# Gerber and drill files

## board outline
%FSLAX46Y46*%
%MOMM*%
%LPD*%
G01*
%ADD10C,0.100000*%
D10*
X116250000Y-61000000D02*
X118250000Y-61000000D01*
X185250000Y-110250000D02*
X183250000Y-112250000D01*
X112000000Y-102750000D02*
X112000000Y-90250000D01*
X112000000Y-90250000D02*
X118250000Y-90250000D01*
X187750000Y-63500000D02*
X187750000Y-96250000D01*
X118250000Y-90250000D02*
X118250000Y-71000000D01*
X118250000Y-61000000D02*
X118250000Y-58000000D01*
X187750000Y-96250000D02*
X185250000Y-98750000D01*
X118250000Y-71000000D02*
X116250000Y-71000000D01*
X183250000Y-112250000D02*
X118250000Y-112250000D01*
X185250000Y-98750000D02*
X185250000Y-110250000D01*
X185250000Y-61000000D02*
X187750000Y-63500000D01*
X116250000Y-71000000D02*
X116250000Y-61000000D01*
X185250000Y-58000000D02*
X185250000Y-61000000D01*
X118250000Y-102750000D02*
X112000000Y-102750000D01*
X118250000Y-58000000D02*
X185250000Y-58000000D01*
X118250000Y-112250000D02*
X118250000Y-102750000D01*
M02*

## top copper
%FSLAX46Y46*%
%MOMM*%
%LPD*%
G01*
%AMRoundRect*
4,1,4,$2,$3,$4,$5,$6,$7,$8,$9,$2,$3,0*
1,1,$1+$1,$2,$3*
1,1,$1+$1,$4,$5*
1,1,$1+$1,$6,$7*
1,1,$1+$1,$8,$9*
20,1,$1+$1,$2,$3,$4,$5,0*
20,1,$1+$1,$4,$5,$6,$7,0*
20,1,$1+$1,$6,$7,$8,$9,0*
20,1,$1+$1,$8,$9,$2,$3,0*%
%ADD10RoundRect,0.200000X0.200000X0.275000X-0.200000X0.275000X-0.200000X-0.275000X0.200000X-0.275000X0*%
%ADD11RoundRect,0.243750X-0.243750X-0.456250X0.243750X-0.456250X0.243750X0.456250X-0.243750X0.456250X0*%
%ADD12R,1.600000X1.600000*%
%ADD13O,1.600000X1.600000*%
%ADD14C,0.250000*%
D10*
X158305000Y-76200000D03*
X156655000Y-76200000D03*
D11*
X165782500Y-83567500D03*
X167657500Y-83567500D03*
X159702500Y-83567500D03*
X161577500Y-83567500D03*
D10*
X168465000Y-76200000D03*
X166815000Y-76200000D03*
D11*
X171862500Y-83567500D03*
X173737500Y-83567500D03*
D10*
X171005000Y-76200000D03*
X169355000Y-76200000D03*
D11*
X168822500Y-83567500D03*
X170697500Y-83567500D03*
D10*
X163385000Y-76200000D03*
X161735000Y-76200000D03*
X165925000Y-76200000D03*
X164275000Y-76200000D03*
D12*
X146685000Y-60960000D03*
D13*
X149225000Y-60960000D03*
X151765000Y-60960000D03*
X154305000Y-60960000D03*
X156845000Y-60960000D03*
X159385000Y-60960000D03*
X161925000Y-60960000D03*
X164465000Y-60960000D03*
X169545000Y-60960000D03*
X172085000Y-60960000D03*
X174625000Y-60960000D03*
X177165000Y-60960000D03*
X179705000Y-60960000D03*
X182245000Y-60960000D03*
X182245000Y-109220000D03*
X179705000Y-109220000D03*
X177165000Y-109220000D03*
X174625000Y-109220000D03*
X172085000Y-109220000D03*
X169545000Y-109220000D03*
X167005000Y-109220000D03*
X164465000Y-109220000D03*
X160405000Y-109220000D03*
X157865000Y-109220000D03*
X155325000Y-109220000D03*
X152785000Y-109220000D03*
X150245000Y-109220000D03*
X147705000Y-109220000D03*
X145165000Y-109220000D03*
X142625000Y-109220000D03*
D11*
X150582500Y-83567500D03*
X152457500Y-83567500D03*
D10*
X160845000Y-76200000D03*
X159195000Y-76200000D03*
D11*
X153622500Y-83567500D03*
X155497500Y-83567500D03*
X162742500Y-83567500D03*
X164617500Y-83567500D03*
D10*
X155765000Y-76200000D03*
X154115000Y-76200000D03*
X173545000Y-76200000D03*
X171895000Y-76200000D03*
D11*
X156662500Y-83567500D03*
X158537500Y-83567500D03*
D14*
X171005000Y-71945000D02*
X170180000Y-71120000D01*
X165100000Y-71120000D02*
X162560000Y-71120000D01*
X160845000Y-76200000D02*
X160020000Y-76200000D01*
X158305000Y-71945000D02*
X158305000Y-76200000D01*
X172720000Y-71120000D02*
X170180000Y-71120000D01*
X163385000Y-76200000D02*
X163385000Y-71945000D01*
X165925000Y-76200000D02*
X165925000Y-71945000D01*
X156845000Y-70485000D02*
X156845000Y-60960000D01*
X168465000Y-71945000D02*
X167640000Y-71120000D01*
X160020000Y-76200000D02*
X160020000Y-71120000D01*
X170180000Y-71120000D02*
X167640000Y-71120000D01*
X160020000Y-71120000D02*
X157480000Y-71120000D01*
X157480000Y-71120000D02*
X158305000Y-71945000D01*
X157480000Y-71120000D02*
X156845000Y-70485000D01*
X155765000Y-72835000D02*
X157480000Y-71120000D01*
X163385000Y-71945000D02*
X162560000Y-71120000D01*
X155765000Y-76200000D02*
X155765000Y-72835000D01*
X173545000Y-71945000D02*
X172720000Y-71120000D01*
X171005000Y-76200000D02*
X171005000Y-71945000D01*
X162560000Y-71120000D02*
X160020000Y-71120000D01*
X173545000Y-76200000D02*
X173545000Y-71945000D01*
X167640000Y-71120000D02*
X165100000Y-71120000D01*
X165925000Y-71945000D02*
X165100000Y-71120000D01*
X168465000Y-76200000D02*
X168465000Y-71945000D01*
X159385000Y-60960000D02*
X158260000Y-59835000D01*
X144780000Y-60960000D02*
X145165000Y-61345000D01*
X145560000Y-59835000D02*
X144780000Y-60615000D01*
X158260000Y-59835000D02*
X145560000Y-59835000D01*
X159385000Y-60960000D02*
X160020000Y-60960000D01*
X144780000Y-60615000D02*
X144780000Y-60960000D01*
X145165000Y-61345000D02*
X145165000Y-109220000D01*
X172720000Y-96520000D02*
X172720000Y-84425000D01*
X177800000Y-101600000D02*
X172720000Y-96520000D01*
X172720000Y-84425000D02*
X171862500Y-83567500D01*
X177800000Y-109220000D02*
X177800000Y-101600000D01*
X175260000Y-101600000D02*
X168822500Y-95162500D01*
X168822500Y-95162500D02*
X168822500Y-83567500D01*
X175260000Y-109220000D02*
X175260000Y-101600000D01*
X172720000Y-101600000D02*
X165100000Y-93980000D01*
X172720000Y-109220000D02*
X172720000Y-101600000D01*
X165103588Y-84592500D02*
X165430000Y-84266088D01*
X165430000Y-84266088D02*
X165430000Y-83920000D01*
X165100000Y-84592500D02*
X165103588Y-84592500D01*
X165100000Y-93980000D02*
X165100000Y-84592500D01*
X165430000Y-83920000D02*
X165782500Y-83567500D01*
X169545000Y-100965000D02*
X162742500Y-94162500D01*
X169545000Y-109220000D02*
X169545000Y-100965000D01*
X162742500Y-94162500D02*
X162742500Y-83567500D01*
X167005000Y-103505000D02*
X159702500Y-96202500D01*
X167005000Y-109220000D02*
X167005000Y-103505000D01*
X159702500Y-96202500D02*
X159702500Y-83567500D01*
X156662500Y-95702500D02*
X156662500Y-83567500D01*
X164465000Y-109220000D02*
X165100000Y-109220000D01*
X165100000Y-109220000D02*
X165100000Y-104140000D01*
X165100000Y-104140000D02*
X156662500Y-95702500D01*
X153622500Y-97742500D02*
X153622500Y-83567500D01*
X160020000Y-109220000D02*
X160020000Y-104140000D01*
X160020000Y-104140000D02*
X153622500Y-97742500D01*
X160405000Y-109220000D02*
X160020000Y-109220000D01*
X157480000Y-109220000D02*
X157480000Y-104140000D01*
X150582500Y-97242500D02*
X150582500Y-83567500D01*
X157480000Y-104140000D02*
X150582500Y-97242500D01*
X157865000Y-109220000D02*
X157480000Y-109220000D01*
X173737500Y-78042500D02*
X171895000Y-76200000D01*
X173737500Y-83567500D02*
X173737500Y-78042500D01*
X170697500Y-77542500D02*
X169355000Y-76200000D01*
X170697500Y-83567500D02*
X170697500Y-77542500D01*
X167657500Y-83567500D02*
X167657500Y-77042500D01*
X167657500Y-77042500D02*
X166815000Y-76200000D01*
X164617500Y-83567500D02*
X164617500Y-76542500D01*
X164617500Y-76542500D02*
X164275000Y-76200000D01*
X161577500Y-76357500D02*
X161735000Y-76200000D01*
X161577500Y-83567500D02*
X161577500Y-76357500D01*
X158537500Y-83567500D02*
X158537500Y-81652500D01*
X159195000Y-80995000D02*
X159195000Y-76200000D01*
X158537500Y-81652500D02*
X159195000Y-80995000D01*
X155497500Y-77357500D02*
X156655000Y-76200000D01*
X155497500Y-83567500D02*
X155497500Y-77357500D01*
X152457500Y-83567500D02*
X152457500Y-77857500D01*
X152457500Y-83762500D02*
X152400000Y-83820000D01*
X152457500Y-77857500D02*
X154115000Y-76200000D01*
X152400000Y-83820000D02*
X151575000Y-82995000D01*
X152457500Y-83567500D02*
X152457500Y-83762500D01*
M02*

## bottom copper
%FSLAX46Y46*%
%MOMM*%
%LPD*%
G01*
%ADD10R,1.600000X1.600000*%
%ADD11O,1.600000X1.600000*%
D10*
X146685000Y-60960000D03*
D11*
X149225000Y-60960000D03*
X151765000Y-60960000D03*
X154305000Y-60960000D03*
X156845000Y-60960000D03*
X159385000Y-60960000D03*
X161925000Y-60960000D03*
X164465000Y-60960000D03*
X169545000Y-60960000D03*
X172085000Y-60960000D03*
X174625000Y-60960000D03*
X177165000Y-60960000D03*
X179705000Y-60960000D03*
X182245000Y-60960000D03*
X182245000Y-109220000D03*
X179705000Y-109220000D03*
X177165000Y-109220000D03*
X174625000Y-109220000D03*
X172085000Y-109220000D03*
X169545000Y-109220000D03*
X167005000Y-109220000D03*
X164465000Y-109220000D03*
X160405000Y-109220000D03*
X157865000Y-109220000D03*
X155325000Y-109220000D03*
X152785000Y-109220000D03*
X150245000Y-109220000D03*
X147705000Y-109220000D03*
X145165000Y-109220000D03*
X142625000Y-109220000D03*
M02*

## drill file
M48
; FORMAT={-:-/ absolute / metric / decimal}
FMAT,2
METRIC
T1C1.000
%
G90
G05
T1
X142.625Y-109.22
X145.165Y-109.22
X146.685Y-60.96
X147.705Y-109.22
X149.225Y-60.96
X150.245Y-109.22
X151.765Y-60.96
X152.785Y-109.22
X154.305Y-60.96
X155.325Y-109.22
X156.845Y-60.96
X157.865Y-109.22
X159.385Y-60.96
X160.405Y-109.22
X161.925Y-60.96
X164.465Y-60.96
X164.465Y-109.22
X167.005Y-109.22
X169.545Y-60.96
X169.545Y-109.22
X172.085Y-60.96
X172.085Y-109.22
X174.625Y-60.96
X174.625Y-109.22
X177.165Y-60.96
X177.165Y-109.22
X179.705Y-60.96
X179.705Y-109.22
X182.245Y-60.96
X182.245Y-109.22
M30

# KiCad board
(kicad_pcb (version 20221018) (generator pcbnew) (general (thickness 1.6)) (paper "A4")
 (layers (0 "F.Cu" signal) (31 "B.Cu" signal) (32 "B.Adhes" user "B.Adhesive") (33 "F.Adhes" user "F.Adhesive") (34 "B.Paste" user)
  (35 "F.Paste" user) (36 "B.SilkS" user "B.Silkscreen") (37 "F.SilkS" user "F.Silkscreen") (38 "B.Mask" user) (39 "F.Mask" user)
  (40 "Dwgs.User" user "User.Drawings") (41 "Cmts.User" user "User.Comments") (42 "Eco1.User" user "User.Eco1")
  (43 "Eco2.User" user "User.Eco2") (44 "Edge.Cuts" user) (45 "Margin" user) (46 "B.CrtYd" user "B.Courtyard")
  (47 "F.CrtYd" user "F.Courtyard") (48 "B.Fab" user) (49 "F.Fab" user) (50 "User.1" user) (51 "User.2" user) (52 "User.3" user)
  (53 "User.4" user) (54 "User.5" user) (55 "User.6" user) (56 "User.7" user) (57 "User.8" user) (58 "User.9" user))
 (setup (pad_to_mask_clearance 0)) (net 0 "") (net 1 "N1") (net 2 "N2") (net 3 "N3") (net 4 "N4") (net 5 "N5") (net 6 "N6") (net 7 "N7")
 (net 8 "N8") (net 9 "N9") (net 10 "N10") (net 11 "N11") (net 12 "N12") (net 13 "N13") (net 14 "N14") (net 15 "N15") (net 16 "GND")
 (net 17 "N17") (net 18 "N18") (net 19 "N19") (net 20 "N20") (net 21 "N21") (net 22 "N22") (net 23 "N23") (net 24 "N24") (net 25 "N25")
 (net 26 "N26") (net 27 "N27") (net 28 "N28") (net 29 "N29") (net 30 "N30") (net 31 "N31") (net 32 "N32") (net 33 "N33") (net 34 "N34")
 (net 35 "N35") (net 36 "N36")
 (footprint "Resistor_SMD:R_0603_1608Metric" (layer "F.Cu") (at 157.48 76.2 180)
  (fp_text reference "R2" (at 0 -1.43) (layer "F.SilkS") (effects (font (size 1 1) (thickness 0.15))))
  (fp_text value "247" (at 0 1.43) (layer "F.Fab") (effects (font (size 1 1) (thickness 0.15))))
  (pad "1" smd roundrect (at -0.825 0 180) (size 0.8 0.95) (layers "F.Cu" "F.Paste" "F.Mask") (roundrect_rratio 0.25) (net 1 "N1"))
  (pad "2" smd roundrect (at 0.825 0 180) (size 0.8 0.95) (layers "F.Cu" "F.Paste" "F.Mask") (roundrect_rratio 0.25) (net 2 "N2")))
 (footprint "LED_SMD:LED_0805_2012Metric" (layer "F.Cu") (at 166.72 83.5675)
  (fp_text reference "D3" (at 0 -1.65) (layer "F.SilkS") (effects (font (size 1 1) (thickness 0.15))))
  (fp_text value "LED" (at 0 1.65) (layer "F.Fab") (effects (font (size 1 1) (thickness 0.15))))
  (pad "1" smd roundrect (at -0.9375 0) (size 0.975 1.4) (layers "F.Cu" "F.Paste" "F.Mask") (roundrect_rratio 0.25) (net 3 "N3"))
  (pad "2" smd roundrect (at 0.9375 0) (size 0.975 1.4) (layers "F.Cu" "F.Paste" "F.Mask") (roundrect_rratio 0.25) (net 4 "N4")))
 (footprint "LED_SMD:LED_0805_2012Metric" (layer "F.Cu") (at 160.64 83.5675)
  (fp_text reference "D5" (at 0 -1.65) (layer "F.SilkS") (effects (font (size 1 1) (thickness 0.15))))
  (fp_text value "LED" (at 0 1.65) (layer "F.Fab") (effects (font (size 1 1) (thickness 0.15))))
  (pad "1" smd roundrect (at -0.9375 0) (size 0.975 1.4) (layers "F.Cu" "F.Paste" "F.Mask") (roundrect_rratio 0.25) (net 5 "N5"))
  (pad "2" smd roundrect (at 0.9375 0) (size 0.975 1.4) (layers "F.Cu" "F.Paste" "F.Mask") (roundrect_rratio 0.25) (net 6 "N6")))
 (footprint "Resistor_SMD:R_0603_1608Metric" (layer "F.Cu") (at 167.64 76.2 180)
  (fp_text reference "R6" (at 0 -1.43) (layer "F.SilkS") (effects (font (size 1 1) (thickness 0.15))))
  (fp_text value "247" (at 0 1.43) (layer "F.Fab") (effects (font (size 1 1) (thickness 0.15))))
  (pad "1" smd roundrect (at -0.825 0 180) (size 0.8 0.95) (layers "F.Cu" "F.Paste" "F.Mask") (roundrect_rratio 0.25) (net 1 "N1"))
  (pad "2" smd roundrect (at 0.825 0 180) (size 0.8 0.95) (layers "F.Cu" "F.Paste" "F.Mask") (roundrect_rratio 0.25) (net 4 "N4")))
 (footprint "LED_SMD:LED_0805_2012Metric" (layer "F.Cu") (at 172.8 83.5675)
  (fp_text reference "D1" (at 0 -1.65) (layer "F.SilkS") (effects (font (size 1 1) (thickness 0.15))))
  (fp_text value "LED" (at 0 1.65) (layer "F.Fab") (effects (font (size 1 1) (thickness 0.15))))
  (pad "1" smd roundrect (at -0.9375 0) (size 0.975 1.4) (layers "F.Cu" "F.Paste" "F.Mask") (roundrect_rratio 0.25) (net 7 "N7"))
  (pad "2" smd roundrect (at 0.9375 0) (size 0.975 1.4) (layers "F.Cu" "F.Paste" "F.Mask") (roundrect_rratio 0.25) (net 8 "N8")))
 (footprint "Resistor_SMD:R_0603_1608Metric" (layer "F.Cu") (at 170.18 76.2 180)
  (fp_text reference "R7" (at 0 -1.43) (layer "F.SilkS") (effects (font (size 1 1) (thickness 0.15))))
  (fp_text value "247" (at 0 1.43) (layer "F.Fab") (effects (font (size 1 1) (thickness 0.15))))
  (pad "1" smd roundrect (at -0.825 0 180) (size 0.8 0.95) (layers "F.Cu" "F.Paste" "F.Mask") (roundrect_rratio 0.25) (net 1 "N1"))
  (pad "2" smd roundrect (at 0.825 0 180) (size 0.8 0.95) (layers "F.Cu" "F.Paste" "F.Mask") (roundrect_rratio 0.25) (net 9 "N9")))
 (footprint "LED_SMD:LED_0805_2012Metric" (layer "F.Cu") (at 169.76 83.5675)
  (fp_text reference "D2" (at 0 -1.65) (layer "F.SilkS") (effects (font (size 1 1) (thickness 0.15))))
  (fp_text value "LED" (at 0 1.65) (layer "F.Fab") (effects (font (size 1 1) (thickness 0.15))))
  (pad "1" smd roundrect (at -0.9375 0) (size 0.975 1.4) (layers "F.Cu" "F.Paste" "F.Mask") (roundrect_rratio 0.25) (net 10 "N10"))
  (pad "2" smd roundrect (at 0.9375 0) (size 0.975 1.4) (layers "F.Cu" "F.Paste" "F.Mask") (roundrect_rratio 0.25) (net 9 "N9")))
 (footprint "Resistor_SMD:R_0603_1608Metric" (layer "F.Cu") (at 162.56 76.2 180)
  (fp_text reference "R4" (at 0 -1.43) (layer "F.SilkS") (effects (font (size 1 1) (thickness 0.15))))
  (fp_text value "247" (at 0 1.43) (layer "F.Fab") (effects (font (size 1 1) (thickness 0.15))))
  (pad "1" smd roundrect (at -0.825 0 180) (size 0.8 0.95) (layers "F.Cu" "F.Paste" "F.Mask") (roundrect_rratio 0.25) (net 1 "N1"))
  (pad "2" smd roundrect (at 0.825 0 180) (size 0.8 0.95) (layers "F.Cu" "F.Paste" "F.Mask") (roundrect_rratio 0.25) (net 6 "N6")))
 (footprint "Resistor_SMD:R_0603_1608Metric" (layer "F.Cu") (at 165.1 76.2 180)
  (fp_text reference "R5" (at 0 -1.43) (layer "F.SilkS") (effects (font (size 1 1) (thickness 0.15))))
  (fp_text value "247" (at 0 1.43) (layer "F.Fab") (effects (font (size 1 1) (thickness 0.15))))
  (pad "1" smd roundrect (at -0.825 0 180) (size 0.8 0.95) (layers "F.Cu" "F.Paste" "F.Mask") (roundrect_rratio 0.25) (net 1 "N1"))
  (pad "2" smd roundrect (at 0.825 0 180) (size 0.8 0.95) (layers "F.Cu" "F.Paste" "F.Mask") (roundrect_rratio 0.25) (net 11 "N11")))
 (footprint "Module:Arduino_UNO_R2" (layer "F.Cu") (at 146.685 60.96)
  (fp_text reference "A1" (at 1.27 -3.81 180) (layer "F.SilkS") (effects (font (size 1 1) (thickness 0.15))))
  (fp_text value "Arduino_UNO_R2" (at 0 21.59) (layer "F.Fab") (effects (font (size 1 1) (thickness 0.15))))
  (pad "1" thru_hole rect (at 0 0 90) (size 1.6 1.6) (drill 1) (layers "*.Cu" "*.Mask") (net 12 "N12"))
  (pad "2" thru_hole oval (at 2.54 0 90) (size 1.6 1.6) (drill 1) (layers "*.Cu" "*.Mask") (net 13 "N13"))
  (pad "3" thru_hole oval (at 5.08 0 90) (size 1.6 1.6) (drill 1) (layers "*.Cu" "*.Mask") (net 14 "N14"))
  (pad "4" thru_hole oval (at 7.62 0 90) (size 1.6 1.6) (drill 1) (layers "*.Cu" "*.Mask") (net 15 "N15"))
  (pad "5" thru_hole oval (at 10.16 0 90) (size 1.6 1.6) (drill 1) (layers "*.Cu" "*.Mask") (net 1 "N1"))
  (pad "6" thru_hole oval (at 12.7 0 90) (size 1.6 1.6) (drill 1) (layers "*.Cu" "*.Mask") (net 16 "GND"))
  (pad "7" thru_hole oval (at 15.24 0 90) (size 1.6 1.6) (drill 1) (layers "*.Cu" "*.Mask") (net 16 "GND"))
  (pad "8" thru_hole oval (at 17.78 0 90) (size 1.6 1.6) (drill 1) (layers "*.Cu" "*.Mask") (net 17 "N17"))
  (pad "9" thru_hole oval (at 22.86 0 90) (size 1.6 1.6) (drill 1) (layers "*.Cu" "*.Mask") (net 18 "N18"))
  (pad "10" thru_hole oval (at 25.4 0 90) (size 1.6 1.6) (drill 1) (layers "*.Cu" "*.Mask") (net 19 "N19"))
  (pad "11" thru_hole oval (at 27.94 0 90) (size 1.6 1.6) (drill 1) (layers "*.Cu" "*.Mask") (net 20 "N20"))
  (pad "12" thru_hole oval (at 30.48 0 90) (size 1.6 1.6) (drill 1) (layers "*.Cu" "*.Mask") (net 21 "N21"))
  (pad "13" thru_hole oval (at 33.02 0 90) (size 1.6 1.6) (drill 1) (layers "*.Cu" "*.Mask") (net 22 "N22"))
  (pad "14" thru_hole oval (at 35.56 0 90) (size 1.6 1.6) (drill 1) (layers "*.Cu" "*.Mask") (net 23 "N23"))
  (pad "15" thru_hole oval (at 35.56 48.26 90) (size 1.6 1.6) (drill 1) (layers "*.Cu" "*.Mask") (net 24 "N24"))
  (pad "16" thru_hole oval (at 33.02 48.26 90) (size 1.6 1.6) (drill 1) (layers "*.Cu" "*.Mask") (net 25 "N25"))
  (pad "17" thru_hole oval (at 30.48 48.26 90) (size 1.6 1.6) (drill 1) (layers "*.Cu" "*.Mask") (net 7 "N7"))
  (pad "18" thru_hole oval (at 27.94 48.26 90) (size 1.6 1.6) (drill 1) (layers "*.Cu" "*.Mask") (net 10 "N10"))
  (pad "19" thru_hole oval (at 25.4 48.26 90) (size 1.6 1.6) (drill 1) (layers "*.Cu" "*.Mask") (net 3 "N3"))
  (pad "20" thru_hole oval (at 22.86 48.26 90) (size 1.6 1.6) (drill 1) (layers "*.Cu" "*.Mask") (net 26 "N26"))
  (pad "21" thru_hole oval (at 20.32 48.26 90) (size 1.6 1.6) (drill 1) (layers "*.Cu" "*.Mask") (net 5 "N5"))
  (pad "22" thru_hole oval (at 17.78 48.26 90) (size 1.6 1.6) (drill 1) (layers "*.Cu" "*.Mask") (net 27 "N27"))
  (pad "23" thru_hole oval (at 13.72 48.26 90) (size 1.6 1.6) (drill 1) (layers "*.Cu" "*.Mask") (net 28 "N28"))
  (pad "24" thru_hole oval (at 11.18 48.26 90) (size 1.6 1.6) (drill 1) (layers "*.Cu" "*.Mask") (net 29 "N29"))
  (pad "25" thru_hole oval (at 8.64 48.26 90) (size 1.6 1.6) (drill 1) (layers "*.Cu" "*.Mask") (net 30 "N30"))
  (pad "26" thru_hole oval (at 6.1 48.26 90) (size 1.6 1.6) (drill 1) (layers "*.Cu" "*.Mask") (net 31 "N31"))
  (pad "27" thru_hole oval (at 3.56 48.26 90) (size 1.6 1.6) (drill 1) (layers "*.Cu" "*.Mask") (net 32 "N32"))
  (pad "28" thru_hole oval (at 1.02 48.26 90) (size 1.6 1.6) (drill 1) (layers "*.Cu" "*.Mask") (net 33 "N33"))
  (pad "29" thru_hole oval (at -1.52 48.26 90) (size 1.6 1.6) (drill 1) (layers "*.Cu" "*.Mask") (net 16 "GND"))
  (pad "30" thru_hole oval (at -4.06 48.26 90) (size 1.6 1.6) (drill 1) (layers "*.Cu" "*.Mask") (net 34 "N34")))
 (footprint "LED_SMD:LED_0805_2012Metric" (layer "F.Cu") (at 151.52 83.5675)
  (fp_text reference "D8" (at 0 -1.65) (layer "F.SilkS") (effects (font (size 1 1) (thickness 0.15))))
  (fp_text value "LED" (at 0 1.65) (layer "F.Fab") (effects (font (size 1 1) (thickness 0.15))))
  (pad "1" smd roundrect (at -0.9375 0) (size 0.975 1.4) (layers "F.Cu" "F.Paste" "F.Mask") (roundrect_rratio 0.25) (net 29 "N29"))
  (pad "2" smd roundrect (at 0.9375 0) (size 0.975 1.4) (layers "F.Cu" "F.Paste" "F.Mask") (roundrect_rratio 0.25) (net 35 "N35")))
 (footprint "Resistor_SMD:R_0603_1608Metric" (layer "F.Cu") (at 160.02 76.2 180)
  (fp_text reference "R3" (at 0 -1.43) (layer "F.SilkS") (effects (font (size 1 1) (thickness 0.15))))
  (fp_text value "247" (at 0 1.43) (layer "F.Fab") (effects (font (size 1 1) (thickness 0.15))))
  (pad "1" smd roundrect (at -0.825 0 180) (size 0.8 0.95) (layers "F.Cu" "F.Paste" "F.Mask") (roundrect_rratio 0.25) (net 1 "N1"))
  (pad "2" smd roundrect (at 0.825 0 180) (size 0.8 0.95) (layers "F.Cu" "F.Paste" "F.Mask") (roundrect_rratio 0.25) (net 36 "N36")))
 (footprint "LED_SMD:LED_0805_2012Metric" (layer "F.Cu") (at 154.56 83.5675)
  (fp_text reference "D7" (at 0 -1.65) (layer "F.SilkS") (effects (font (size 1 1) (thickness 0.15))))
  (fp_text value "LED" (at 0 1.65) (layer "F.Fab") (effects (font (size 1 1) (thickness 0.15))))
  (pad "1" smd roundrect (at -0.9375 0) (size 0.975 1.4) (layers "F.Cu" "F.Paste" "F.Mask") (roundrect_rratio 0.25) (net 28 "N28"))
  (pad "2" smd roundrect (at 0.9375 0) (size 0.975 1.4) (layers "F.Cu" "F.Paste" "F.Mask") (roundrect_rratio 0.25) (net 2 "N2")))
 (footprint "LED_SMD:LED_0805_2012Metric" (layer "F.Cu") (at 163.68 83.5675)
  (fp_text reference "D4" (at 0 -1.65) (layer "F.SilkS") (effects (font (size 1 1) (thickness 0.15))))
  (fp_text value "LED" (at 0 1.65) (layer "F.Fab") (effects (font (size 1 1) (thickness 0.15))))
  (pad "1" smd roundrect (at -0.9375 0) (size 0.975 1.4) (layers "F.Cu" "F.Paste" "F.Mask") (roundrect_rratio 0.25) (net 26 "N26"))
  (pad "2" smd roundrect (at 0.9375 0) (size 0.975 1.4) (layers "F.Cu" "F.Paste" "F.Mask") (roundrect_rratio 0.25) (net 11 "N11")))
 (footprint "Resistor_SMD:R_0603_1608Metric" (layer "F.Cu") (at 154.94 76.2 180)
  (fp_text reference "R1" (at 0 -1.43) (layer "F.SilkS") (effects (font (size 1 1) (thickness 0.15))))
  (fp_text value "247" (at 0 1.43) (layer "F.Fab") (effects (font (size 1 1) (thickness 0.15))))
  (pad "1" smd roundrect (at -0.825 0 180) (size 0.8 0.95) (layers "F.Cu" "F.Paste" "F.Mask") (roundrect_rratio 0.25) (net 1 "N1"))
  (pad "2" smd roundrect (at 0.825 0 180) (size 0.8 0.95) (layers "F.Cu" "F.Paste" "F.Mask") (roundrect_rratio 0.25) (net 35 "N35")))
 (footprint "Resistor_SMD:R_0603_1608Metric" (layer "F.Cu") (at 172.72 76.2 180)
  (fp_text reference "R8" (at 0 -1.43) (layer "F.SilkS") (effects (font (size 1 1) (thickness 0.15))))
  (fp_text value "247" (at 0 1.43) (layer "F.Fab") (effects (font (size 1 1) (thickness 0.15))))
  (pad "1" smd roundrect (at -0.825 0 180) (size 0.8 0.95) (layers "F.Cu" "F.Paste" "F.Mask") (roundrect_rratio 0.25) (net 1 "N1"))
  (pad "2" smd roundrect (at 0.825 0 180) (size 0.8 0.95) (layers "F.Cu" "F.Paste" "F.Mask") (roundrect_rratio 0.25) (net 8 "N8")))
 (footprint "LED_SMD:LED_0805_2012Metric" (layer "F.Cu") (at 157.6 83.5675)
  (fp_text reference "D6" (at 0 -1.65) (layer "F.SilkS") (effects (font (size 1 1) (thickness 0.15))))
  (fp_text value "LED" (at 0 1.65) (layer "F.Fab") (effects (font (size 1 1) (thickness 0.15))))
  (pad "1" smd roundrect (at -0.9375 0) (size 0.975 1.4) (layers "F.Cu" "F.Paste" "F.Mask") (roundrect_rratio 0.25) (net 27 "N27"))
  (pad "2" smd roundrect (at 0.9375 0) (size 0.975 1.4) (layers "F.Cu" "F.Paste" "F.Mask") (roundrect_rratio 0.25) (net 36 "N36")))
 (gr_line (start 116.25 61) (end 118.25 61) (stroke (width 0.1) (type default)) (layer "Edge.Cuts"))
 (gr_line (start 185.25 110.25) (end 183.25 112.25) (stroke (width 0.1) (type default)) (layer "Edge.Cuts"))
 (gr_line (start 112 102.75) (end 112 90.25) (stroke (width 0.1) (type default)) (layer "Edge.Cuts"))
 (gr_line (start 112 90.25) (end 118.25 90.25) (stroke (width 0.1) (type default)) (layer "Edge.Cuts"))
 (gr_line (start 187.75 63.5) (end 187.75 96.25) (stroke (width 0.1) (type default)) (layer "Edge.Cuts"))
 (gr_line (start 118.25 90.25) (end 118.25 71) (stroke (width 0.1) (type default)) (layer "Edge.Cuts"))
 (gr_line (start 118.25 61) (end 118.25 58) (stroke (width 0.1) (type default)) (layer "Edge.Cuts"))
 (gr_line (start 187.75 96.25) (end 185.25 98.75) (stroke (width 0.1) (type default)) (layer "Edge.Cuts"))
 (gr_line (start 118.25 71) (end 116.25 71) (stroke (width 0.1) (type default)) (layer "Edge.Cuts"))
 (gr_line (start 183.25 112.25) (end 118.25 112.25) (stroke (width 0.1) (type default)) (layer "Edge.Cuts"))
 (gr_line (start 185.25 98.75) (end 185.25 110.25) (stroke (width 0.1) (type default)) (layer "Edge.Cuts"))
 (gr_line (start 185.25 61) (end 187.75 63.5) (stroke (width 0.1) (type default)) (layer "Edge.Cuts"))
 (gr_line (start 116.25 71) (end 116.25 61) (stroke (width 0.1) (type default)) (layer "Edge.Cuts"))
 (gr_line (start 185.25 58) (end 185.25 61) (stroke (width 0.1) (type default)) (layer "Edge.Cuts"))
 (gr_line (start 118.25 102.75) (end 112 102.75) (stroke (width 0.1) (type default)) (layer "Edge.Cuts"))
 (gr_line (start 118.25 58) (end 185.25 58) (stroke (width 0.1) (type default)) (layer "Edge.Cuts"))
 (gr_line (start 118.25 112.25) (end 118.25 102.75) (stroke (width 0.1) (type default)) (layer "Edge.Cuts"))
 (segment (start 171.005 71.945) (end 170.18 71.12) (width 0.25) (layer "F.Cu") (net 1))
 (segment (start 165.1 71.12) (end 162.56 71.12) (width 0.25) (layer "F.Cu") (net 1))
 (segment (start 160.845 76.2) (end 160.02 76.2) (width 0.25) (layer "F.Cu") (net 1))
 (segment (start 158.305 71.945) (end 158.305 76.2) (width 0.25) (layer "F.Cu") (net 1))
 (segment (start 172.72 71.12) (end 170.18 71.12) (width 0.25) (layer "F.Cu") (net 1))
 (segment (start 163.385 76.2) (end 163.385 71.945) (width 0.25) (layer "F.Cu") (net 1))
 (segment (start 165.925 76.2) (end 165.925 71.945) (width 0.25) (layer "F.Cu") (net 1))
 (segment (start 156.845 70.485) (end 156.845 60.96) (width 0.25) (layer "F.Cu") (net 1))
 (segment (start 168.465 71.945) (end 167.64 71.12) (width 0.25) (layer "F.Cu") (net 1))
 (segment (start 160.02 76.2) (end 160.02 71.12) (width 0.25) (layer "F.Cu") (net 1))
 (segment (start 170.18 71.12) (end 167.64 71.12) (width 0.25) (layer "F.Cu") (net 1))
 (segment (start 160.02 71.12) (end 157.48 71.12) (width 0.25) (layer "F.Cu") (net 1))
 (segment (start 157.48 71.12) (end 158.305 71.945) (width 0.25) (layer "F.Cu") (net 1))
 (segment (start 157.48 71.12) (end 156.845 70.485) (width 0.25) (layer "F.Cu") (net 1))
 (segment (start 155.765 72.835) (end 157.48 71.12) (width 0.25) (layer "F.Cu") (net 1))
 (segment (start 163.385 71.945) (end 162.56 71.12) (width 0.25) (layer "F.Cu") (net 1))
 (segment (start 155.765 76.2) (end 155.765 72.835) (width 0.25) (layer "F.Cu") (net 1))
 (segment (start 173.545 71.945) (end 172.72 71.12) (width 0.25) (layer "F.Cu") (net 1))
 (segment (start 171.005 76.2) (end 171.005 71.945) (width 0.25) (layer "F.Cu") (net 1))
 (segment (start 162.56 71.12) (end 160.02 71.12) (width 0.25) (layer "F.Cu") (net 1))
 (segment (start 173.545 76.2) (end 173.545 71.945) (width 0.25) (layer "F.Cu") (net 1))
 (segment (start 167.64 71.12) (end 165.1 71.12) (width 0.25) (layer "F.Cu") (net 1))
 (segment (start 165.925 71.945) (end 165.1 71.12) (width 0.25) (layer "F.Cu") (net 1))
 (segment (start 168.465 76.2) (end 168.465 71.945) (width 0.25) (layer "F.Cu") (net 1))
 (segment (start 159.385 60.96) (end 158.26 59.835) (width 0.25) (layer "F.Cu") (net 16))
 (segment (start 144.78 60.96) (end 145.165 61.345) (width 0.25) (layer "F.Cu") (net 16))
 (segment (start 145.56 59.835) (end 144.78 60.615) (width 0.25) (layer "F.Cu") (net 16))
 (segment (start 158.26 59.835) (end 145.56 59.835) (width 0.25) (layer "F.Cu") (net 16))
 (segment (start 159.385 60.96) (end 160.02 60.96) (width 0.25) (layer "F.Cu") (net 16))
 (segment (start 144.78 60.615) (end 144.78 60.96) (width 0.25) (layer "F.Cu") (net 16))
 (segment (start 145.165 61.345) (end 145.165 109.22) (width 0.25) (layer "F.Cu") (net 16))
 (segment (start 172.72 96.52) (end 172.72 84.425) (width 0.25) (layer "F.Cu") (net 7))
 (segment (start 177.8 101.6) (end 172.72 96.52) (width 0.25) (layer "F.Cu") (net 7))
 (segment (start 172.72 84.425) (end 171.8625 83.5675) (width 0.25) (layer "F.Cu") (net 7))
 (segment (start 177.8 109.22) (end 177.8 101.6) (width 0.25) (layer "F.Cu") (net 7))
 (segment (start 175.26 101.6) (end 168.8225 95.1625) (width 0.25) (layer "F.Cu") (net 10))
 (segment (start 168.8225 95.1625) (end 168.8225 83.5675) (width 0.25) (layer "F.Cu") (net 10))
 (segment (start 175.26 109.22) (end 175.26 101.6) (width 0.25) (layer "F.Cu") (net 10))
 (segment (start 172.72 101.6) (end 165.1 93.98) (width 0.25) (layer "F.Cu") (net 3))
 (segment (start 172.72 109.22) (end 172.72 101.6) (width 0.25) (layer "F.Cu") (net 3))
 (segment (start 165.103588 84.5925) (end 165.43 84.266088) (width 0.25) (layer "F.Cu") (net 3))
 (segment (start 165.43 84.266088) (end 165.43 83.92) (width 0.25) (layer "F.Cu") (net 3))
 (segment (start 165.1 84.5925) (end 165.103588 84.5925) (width 0.25) (layer "F.Cu") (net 3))
 (segment (start 165.1 93.98) (end 165.1 84.5925) (width 0.25) (layer "F.Cu") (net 3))
 (segment (start 165.43 83.92) (end 165.7825 83.5675) (width 0.25) (layer "F.Cu") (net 3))
 (segment (start 169.545 100.965) (end 162.7425 94.1625) (width 0.25) (layer "F.Cu") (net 26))
 (segment (start 169.545 109.22) (end 169.545 100.965) (width 0.25) (layer "F.Cu") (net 26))
 (segment (start 162.7425 94.1625) (end 162.7425 83.5675) (width 0.25) (layer "F.Cu") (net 26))
 (segment (start 167.005 103.505) (end 159.7025 96.2025) (width 0.25) (layer "F.Cu") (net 5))
 (segment (start 167.005 109.22) (end 167.005 103.505) (width 0.25) (layer "F.Cu") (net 5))
 (segment (start 159.7025 96.2025) (end 159.7025 83.5675) (width 0.25) (layer "F.Cu") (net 5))
 (segment (start 156.6625 95.7025) (end 156.6625 83.5675) (width 0.25) (layer "F.Cu") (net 27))
 (segment (start 164.465 109.22) (end 165.1 109.22) (width 0.25) (layer "F.Cu") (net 27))
 (segment (start 165.1 109.22) (end 165.1 104.14) (width 0.25) (layer "F.Cu") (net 27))
 (segment (start 165.1 104.14) (end 156.6625 95.7025) (width 0.25) (layer "F.Cu") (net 27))
 (segment (start 153.6225 97.7425) (end 153.6225 83.5675) (width 0.25) (layer "F.Cu") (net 28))
 (segment (start 160.02 109.22) (end 160.02 104.14) (width 0.25) (layer "F.Cu") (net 28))
 (segment (start 160.02 104.14) (end 153.6225 97.7425) (width 0.25) (layer "F.Cu") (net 28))
 (segment (start 160.405 109.22) (end 160.02 109.22) (width 0.25) (layer "F.Cu") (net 28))
 (segment (start 157.48 109.22) (end 157.48 104.14) (width 0.25) (layer "F.Cu") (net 29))
 (segment (start 150.5825 97.2425) (end 150.5825 83.5675) (width 0.25) (layer "F.Cu") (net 29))
 (segment (start 157.48 104.14) (end 150.5825 97.2425) (width 0.25) (layer "F.Cu") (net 29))
 (segment (start 157.865 109.22) (end 157.48 109.22) (width 0.25) (layer "F.Cu") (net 29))
 (segment (start 173.7375 78.0425) (end 171.895 76.2) (width 0.25) (layer "F.Cu") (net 8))
 (segment (start 173.7375 83.5675) (end 173.7375 78.0425) (width 0.25) (layer "F.Cu") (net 8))
 (segment (start 170.6975 77.5425) (end 169.355 76.2) (width 0.25) (layer "F.Cu") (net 9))
 (segment (start 170.6975 83.5675) (end 170.6975 77.5425) (width 0.25) (layer "F.Cu") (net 9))
 (segment (start 167.6575 83.5675) (end 167.6575 77.0425) (width 0.25) (layer "F.Cu") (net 4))
 (segment (start 167.6575 77.0425) (end 166.815 76.2) (width 0.25) (layer "F.Cu") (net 4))
 (segment (start 164.6175 83.5675) (end 164.6175 76.5425) (width 0.25) (layer "F.Cu") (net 11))
 (segment (start 164.6175 76.5425) (end 164.275 76.2) (width 0.25) (layer "F.Cu") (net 11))
 (segment (start 161.5775 76.3575) (end 161.735 76.2) (width 0.25) (layer "F.Cu") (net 6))
 (segment (start 161.5775 83.5675) (end 161.5775 76.3575) (width 0.25) (layer "F.Cu") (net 6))
 (segment (start 158.5375 83.5675) (end 158.5375 81.6525) (width 0.25) (layer "F.Cu") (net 36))
 (segment (start 159.195 80.995) (end 159.195 76.2) (width 0.25) (layer "F.Cu") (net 36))
 (segment (start 158.5375 81.6525) (end 159.195 80.995) (width 0.25) (layer "F.Cu") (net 36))
 (segment (start 155.4975 77.3575) (end 156.655 76.2) (width 0.25) (layer "F.Cu") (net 2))
 (segment (start 155.4975 83.5675) (end 155.4975 77.3575) (width 0.25) (layer "F.Cu") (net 2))
 (segment (start 152.4575 83.5675) (end 152.4575 77.8575) (width 0.25) (layer "F.Cu") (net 35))
 (segment (start 152.4575 83.7625) (end 152.4 83.82) (width 0.25) (layer "F.Cu") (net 35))
 (segment (start 152.4575 77.8575) (end 154.115 76.2) (width 0.25) (layer "F.Cu") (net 35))
 (segment (start 152.4 83.82) (end 151.575 82.995) (width 0.25) (layer "F.Cu") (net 35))
 (segment (start 152.4575 83.5675) (end 152.4575 83.7625) (width 0.25) (layer "F.Cu") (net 35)))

